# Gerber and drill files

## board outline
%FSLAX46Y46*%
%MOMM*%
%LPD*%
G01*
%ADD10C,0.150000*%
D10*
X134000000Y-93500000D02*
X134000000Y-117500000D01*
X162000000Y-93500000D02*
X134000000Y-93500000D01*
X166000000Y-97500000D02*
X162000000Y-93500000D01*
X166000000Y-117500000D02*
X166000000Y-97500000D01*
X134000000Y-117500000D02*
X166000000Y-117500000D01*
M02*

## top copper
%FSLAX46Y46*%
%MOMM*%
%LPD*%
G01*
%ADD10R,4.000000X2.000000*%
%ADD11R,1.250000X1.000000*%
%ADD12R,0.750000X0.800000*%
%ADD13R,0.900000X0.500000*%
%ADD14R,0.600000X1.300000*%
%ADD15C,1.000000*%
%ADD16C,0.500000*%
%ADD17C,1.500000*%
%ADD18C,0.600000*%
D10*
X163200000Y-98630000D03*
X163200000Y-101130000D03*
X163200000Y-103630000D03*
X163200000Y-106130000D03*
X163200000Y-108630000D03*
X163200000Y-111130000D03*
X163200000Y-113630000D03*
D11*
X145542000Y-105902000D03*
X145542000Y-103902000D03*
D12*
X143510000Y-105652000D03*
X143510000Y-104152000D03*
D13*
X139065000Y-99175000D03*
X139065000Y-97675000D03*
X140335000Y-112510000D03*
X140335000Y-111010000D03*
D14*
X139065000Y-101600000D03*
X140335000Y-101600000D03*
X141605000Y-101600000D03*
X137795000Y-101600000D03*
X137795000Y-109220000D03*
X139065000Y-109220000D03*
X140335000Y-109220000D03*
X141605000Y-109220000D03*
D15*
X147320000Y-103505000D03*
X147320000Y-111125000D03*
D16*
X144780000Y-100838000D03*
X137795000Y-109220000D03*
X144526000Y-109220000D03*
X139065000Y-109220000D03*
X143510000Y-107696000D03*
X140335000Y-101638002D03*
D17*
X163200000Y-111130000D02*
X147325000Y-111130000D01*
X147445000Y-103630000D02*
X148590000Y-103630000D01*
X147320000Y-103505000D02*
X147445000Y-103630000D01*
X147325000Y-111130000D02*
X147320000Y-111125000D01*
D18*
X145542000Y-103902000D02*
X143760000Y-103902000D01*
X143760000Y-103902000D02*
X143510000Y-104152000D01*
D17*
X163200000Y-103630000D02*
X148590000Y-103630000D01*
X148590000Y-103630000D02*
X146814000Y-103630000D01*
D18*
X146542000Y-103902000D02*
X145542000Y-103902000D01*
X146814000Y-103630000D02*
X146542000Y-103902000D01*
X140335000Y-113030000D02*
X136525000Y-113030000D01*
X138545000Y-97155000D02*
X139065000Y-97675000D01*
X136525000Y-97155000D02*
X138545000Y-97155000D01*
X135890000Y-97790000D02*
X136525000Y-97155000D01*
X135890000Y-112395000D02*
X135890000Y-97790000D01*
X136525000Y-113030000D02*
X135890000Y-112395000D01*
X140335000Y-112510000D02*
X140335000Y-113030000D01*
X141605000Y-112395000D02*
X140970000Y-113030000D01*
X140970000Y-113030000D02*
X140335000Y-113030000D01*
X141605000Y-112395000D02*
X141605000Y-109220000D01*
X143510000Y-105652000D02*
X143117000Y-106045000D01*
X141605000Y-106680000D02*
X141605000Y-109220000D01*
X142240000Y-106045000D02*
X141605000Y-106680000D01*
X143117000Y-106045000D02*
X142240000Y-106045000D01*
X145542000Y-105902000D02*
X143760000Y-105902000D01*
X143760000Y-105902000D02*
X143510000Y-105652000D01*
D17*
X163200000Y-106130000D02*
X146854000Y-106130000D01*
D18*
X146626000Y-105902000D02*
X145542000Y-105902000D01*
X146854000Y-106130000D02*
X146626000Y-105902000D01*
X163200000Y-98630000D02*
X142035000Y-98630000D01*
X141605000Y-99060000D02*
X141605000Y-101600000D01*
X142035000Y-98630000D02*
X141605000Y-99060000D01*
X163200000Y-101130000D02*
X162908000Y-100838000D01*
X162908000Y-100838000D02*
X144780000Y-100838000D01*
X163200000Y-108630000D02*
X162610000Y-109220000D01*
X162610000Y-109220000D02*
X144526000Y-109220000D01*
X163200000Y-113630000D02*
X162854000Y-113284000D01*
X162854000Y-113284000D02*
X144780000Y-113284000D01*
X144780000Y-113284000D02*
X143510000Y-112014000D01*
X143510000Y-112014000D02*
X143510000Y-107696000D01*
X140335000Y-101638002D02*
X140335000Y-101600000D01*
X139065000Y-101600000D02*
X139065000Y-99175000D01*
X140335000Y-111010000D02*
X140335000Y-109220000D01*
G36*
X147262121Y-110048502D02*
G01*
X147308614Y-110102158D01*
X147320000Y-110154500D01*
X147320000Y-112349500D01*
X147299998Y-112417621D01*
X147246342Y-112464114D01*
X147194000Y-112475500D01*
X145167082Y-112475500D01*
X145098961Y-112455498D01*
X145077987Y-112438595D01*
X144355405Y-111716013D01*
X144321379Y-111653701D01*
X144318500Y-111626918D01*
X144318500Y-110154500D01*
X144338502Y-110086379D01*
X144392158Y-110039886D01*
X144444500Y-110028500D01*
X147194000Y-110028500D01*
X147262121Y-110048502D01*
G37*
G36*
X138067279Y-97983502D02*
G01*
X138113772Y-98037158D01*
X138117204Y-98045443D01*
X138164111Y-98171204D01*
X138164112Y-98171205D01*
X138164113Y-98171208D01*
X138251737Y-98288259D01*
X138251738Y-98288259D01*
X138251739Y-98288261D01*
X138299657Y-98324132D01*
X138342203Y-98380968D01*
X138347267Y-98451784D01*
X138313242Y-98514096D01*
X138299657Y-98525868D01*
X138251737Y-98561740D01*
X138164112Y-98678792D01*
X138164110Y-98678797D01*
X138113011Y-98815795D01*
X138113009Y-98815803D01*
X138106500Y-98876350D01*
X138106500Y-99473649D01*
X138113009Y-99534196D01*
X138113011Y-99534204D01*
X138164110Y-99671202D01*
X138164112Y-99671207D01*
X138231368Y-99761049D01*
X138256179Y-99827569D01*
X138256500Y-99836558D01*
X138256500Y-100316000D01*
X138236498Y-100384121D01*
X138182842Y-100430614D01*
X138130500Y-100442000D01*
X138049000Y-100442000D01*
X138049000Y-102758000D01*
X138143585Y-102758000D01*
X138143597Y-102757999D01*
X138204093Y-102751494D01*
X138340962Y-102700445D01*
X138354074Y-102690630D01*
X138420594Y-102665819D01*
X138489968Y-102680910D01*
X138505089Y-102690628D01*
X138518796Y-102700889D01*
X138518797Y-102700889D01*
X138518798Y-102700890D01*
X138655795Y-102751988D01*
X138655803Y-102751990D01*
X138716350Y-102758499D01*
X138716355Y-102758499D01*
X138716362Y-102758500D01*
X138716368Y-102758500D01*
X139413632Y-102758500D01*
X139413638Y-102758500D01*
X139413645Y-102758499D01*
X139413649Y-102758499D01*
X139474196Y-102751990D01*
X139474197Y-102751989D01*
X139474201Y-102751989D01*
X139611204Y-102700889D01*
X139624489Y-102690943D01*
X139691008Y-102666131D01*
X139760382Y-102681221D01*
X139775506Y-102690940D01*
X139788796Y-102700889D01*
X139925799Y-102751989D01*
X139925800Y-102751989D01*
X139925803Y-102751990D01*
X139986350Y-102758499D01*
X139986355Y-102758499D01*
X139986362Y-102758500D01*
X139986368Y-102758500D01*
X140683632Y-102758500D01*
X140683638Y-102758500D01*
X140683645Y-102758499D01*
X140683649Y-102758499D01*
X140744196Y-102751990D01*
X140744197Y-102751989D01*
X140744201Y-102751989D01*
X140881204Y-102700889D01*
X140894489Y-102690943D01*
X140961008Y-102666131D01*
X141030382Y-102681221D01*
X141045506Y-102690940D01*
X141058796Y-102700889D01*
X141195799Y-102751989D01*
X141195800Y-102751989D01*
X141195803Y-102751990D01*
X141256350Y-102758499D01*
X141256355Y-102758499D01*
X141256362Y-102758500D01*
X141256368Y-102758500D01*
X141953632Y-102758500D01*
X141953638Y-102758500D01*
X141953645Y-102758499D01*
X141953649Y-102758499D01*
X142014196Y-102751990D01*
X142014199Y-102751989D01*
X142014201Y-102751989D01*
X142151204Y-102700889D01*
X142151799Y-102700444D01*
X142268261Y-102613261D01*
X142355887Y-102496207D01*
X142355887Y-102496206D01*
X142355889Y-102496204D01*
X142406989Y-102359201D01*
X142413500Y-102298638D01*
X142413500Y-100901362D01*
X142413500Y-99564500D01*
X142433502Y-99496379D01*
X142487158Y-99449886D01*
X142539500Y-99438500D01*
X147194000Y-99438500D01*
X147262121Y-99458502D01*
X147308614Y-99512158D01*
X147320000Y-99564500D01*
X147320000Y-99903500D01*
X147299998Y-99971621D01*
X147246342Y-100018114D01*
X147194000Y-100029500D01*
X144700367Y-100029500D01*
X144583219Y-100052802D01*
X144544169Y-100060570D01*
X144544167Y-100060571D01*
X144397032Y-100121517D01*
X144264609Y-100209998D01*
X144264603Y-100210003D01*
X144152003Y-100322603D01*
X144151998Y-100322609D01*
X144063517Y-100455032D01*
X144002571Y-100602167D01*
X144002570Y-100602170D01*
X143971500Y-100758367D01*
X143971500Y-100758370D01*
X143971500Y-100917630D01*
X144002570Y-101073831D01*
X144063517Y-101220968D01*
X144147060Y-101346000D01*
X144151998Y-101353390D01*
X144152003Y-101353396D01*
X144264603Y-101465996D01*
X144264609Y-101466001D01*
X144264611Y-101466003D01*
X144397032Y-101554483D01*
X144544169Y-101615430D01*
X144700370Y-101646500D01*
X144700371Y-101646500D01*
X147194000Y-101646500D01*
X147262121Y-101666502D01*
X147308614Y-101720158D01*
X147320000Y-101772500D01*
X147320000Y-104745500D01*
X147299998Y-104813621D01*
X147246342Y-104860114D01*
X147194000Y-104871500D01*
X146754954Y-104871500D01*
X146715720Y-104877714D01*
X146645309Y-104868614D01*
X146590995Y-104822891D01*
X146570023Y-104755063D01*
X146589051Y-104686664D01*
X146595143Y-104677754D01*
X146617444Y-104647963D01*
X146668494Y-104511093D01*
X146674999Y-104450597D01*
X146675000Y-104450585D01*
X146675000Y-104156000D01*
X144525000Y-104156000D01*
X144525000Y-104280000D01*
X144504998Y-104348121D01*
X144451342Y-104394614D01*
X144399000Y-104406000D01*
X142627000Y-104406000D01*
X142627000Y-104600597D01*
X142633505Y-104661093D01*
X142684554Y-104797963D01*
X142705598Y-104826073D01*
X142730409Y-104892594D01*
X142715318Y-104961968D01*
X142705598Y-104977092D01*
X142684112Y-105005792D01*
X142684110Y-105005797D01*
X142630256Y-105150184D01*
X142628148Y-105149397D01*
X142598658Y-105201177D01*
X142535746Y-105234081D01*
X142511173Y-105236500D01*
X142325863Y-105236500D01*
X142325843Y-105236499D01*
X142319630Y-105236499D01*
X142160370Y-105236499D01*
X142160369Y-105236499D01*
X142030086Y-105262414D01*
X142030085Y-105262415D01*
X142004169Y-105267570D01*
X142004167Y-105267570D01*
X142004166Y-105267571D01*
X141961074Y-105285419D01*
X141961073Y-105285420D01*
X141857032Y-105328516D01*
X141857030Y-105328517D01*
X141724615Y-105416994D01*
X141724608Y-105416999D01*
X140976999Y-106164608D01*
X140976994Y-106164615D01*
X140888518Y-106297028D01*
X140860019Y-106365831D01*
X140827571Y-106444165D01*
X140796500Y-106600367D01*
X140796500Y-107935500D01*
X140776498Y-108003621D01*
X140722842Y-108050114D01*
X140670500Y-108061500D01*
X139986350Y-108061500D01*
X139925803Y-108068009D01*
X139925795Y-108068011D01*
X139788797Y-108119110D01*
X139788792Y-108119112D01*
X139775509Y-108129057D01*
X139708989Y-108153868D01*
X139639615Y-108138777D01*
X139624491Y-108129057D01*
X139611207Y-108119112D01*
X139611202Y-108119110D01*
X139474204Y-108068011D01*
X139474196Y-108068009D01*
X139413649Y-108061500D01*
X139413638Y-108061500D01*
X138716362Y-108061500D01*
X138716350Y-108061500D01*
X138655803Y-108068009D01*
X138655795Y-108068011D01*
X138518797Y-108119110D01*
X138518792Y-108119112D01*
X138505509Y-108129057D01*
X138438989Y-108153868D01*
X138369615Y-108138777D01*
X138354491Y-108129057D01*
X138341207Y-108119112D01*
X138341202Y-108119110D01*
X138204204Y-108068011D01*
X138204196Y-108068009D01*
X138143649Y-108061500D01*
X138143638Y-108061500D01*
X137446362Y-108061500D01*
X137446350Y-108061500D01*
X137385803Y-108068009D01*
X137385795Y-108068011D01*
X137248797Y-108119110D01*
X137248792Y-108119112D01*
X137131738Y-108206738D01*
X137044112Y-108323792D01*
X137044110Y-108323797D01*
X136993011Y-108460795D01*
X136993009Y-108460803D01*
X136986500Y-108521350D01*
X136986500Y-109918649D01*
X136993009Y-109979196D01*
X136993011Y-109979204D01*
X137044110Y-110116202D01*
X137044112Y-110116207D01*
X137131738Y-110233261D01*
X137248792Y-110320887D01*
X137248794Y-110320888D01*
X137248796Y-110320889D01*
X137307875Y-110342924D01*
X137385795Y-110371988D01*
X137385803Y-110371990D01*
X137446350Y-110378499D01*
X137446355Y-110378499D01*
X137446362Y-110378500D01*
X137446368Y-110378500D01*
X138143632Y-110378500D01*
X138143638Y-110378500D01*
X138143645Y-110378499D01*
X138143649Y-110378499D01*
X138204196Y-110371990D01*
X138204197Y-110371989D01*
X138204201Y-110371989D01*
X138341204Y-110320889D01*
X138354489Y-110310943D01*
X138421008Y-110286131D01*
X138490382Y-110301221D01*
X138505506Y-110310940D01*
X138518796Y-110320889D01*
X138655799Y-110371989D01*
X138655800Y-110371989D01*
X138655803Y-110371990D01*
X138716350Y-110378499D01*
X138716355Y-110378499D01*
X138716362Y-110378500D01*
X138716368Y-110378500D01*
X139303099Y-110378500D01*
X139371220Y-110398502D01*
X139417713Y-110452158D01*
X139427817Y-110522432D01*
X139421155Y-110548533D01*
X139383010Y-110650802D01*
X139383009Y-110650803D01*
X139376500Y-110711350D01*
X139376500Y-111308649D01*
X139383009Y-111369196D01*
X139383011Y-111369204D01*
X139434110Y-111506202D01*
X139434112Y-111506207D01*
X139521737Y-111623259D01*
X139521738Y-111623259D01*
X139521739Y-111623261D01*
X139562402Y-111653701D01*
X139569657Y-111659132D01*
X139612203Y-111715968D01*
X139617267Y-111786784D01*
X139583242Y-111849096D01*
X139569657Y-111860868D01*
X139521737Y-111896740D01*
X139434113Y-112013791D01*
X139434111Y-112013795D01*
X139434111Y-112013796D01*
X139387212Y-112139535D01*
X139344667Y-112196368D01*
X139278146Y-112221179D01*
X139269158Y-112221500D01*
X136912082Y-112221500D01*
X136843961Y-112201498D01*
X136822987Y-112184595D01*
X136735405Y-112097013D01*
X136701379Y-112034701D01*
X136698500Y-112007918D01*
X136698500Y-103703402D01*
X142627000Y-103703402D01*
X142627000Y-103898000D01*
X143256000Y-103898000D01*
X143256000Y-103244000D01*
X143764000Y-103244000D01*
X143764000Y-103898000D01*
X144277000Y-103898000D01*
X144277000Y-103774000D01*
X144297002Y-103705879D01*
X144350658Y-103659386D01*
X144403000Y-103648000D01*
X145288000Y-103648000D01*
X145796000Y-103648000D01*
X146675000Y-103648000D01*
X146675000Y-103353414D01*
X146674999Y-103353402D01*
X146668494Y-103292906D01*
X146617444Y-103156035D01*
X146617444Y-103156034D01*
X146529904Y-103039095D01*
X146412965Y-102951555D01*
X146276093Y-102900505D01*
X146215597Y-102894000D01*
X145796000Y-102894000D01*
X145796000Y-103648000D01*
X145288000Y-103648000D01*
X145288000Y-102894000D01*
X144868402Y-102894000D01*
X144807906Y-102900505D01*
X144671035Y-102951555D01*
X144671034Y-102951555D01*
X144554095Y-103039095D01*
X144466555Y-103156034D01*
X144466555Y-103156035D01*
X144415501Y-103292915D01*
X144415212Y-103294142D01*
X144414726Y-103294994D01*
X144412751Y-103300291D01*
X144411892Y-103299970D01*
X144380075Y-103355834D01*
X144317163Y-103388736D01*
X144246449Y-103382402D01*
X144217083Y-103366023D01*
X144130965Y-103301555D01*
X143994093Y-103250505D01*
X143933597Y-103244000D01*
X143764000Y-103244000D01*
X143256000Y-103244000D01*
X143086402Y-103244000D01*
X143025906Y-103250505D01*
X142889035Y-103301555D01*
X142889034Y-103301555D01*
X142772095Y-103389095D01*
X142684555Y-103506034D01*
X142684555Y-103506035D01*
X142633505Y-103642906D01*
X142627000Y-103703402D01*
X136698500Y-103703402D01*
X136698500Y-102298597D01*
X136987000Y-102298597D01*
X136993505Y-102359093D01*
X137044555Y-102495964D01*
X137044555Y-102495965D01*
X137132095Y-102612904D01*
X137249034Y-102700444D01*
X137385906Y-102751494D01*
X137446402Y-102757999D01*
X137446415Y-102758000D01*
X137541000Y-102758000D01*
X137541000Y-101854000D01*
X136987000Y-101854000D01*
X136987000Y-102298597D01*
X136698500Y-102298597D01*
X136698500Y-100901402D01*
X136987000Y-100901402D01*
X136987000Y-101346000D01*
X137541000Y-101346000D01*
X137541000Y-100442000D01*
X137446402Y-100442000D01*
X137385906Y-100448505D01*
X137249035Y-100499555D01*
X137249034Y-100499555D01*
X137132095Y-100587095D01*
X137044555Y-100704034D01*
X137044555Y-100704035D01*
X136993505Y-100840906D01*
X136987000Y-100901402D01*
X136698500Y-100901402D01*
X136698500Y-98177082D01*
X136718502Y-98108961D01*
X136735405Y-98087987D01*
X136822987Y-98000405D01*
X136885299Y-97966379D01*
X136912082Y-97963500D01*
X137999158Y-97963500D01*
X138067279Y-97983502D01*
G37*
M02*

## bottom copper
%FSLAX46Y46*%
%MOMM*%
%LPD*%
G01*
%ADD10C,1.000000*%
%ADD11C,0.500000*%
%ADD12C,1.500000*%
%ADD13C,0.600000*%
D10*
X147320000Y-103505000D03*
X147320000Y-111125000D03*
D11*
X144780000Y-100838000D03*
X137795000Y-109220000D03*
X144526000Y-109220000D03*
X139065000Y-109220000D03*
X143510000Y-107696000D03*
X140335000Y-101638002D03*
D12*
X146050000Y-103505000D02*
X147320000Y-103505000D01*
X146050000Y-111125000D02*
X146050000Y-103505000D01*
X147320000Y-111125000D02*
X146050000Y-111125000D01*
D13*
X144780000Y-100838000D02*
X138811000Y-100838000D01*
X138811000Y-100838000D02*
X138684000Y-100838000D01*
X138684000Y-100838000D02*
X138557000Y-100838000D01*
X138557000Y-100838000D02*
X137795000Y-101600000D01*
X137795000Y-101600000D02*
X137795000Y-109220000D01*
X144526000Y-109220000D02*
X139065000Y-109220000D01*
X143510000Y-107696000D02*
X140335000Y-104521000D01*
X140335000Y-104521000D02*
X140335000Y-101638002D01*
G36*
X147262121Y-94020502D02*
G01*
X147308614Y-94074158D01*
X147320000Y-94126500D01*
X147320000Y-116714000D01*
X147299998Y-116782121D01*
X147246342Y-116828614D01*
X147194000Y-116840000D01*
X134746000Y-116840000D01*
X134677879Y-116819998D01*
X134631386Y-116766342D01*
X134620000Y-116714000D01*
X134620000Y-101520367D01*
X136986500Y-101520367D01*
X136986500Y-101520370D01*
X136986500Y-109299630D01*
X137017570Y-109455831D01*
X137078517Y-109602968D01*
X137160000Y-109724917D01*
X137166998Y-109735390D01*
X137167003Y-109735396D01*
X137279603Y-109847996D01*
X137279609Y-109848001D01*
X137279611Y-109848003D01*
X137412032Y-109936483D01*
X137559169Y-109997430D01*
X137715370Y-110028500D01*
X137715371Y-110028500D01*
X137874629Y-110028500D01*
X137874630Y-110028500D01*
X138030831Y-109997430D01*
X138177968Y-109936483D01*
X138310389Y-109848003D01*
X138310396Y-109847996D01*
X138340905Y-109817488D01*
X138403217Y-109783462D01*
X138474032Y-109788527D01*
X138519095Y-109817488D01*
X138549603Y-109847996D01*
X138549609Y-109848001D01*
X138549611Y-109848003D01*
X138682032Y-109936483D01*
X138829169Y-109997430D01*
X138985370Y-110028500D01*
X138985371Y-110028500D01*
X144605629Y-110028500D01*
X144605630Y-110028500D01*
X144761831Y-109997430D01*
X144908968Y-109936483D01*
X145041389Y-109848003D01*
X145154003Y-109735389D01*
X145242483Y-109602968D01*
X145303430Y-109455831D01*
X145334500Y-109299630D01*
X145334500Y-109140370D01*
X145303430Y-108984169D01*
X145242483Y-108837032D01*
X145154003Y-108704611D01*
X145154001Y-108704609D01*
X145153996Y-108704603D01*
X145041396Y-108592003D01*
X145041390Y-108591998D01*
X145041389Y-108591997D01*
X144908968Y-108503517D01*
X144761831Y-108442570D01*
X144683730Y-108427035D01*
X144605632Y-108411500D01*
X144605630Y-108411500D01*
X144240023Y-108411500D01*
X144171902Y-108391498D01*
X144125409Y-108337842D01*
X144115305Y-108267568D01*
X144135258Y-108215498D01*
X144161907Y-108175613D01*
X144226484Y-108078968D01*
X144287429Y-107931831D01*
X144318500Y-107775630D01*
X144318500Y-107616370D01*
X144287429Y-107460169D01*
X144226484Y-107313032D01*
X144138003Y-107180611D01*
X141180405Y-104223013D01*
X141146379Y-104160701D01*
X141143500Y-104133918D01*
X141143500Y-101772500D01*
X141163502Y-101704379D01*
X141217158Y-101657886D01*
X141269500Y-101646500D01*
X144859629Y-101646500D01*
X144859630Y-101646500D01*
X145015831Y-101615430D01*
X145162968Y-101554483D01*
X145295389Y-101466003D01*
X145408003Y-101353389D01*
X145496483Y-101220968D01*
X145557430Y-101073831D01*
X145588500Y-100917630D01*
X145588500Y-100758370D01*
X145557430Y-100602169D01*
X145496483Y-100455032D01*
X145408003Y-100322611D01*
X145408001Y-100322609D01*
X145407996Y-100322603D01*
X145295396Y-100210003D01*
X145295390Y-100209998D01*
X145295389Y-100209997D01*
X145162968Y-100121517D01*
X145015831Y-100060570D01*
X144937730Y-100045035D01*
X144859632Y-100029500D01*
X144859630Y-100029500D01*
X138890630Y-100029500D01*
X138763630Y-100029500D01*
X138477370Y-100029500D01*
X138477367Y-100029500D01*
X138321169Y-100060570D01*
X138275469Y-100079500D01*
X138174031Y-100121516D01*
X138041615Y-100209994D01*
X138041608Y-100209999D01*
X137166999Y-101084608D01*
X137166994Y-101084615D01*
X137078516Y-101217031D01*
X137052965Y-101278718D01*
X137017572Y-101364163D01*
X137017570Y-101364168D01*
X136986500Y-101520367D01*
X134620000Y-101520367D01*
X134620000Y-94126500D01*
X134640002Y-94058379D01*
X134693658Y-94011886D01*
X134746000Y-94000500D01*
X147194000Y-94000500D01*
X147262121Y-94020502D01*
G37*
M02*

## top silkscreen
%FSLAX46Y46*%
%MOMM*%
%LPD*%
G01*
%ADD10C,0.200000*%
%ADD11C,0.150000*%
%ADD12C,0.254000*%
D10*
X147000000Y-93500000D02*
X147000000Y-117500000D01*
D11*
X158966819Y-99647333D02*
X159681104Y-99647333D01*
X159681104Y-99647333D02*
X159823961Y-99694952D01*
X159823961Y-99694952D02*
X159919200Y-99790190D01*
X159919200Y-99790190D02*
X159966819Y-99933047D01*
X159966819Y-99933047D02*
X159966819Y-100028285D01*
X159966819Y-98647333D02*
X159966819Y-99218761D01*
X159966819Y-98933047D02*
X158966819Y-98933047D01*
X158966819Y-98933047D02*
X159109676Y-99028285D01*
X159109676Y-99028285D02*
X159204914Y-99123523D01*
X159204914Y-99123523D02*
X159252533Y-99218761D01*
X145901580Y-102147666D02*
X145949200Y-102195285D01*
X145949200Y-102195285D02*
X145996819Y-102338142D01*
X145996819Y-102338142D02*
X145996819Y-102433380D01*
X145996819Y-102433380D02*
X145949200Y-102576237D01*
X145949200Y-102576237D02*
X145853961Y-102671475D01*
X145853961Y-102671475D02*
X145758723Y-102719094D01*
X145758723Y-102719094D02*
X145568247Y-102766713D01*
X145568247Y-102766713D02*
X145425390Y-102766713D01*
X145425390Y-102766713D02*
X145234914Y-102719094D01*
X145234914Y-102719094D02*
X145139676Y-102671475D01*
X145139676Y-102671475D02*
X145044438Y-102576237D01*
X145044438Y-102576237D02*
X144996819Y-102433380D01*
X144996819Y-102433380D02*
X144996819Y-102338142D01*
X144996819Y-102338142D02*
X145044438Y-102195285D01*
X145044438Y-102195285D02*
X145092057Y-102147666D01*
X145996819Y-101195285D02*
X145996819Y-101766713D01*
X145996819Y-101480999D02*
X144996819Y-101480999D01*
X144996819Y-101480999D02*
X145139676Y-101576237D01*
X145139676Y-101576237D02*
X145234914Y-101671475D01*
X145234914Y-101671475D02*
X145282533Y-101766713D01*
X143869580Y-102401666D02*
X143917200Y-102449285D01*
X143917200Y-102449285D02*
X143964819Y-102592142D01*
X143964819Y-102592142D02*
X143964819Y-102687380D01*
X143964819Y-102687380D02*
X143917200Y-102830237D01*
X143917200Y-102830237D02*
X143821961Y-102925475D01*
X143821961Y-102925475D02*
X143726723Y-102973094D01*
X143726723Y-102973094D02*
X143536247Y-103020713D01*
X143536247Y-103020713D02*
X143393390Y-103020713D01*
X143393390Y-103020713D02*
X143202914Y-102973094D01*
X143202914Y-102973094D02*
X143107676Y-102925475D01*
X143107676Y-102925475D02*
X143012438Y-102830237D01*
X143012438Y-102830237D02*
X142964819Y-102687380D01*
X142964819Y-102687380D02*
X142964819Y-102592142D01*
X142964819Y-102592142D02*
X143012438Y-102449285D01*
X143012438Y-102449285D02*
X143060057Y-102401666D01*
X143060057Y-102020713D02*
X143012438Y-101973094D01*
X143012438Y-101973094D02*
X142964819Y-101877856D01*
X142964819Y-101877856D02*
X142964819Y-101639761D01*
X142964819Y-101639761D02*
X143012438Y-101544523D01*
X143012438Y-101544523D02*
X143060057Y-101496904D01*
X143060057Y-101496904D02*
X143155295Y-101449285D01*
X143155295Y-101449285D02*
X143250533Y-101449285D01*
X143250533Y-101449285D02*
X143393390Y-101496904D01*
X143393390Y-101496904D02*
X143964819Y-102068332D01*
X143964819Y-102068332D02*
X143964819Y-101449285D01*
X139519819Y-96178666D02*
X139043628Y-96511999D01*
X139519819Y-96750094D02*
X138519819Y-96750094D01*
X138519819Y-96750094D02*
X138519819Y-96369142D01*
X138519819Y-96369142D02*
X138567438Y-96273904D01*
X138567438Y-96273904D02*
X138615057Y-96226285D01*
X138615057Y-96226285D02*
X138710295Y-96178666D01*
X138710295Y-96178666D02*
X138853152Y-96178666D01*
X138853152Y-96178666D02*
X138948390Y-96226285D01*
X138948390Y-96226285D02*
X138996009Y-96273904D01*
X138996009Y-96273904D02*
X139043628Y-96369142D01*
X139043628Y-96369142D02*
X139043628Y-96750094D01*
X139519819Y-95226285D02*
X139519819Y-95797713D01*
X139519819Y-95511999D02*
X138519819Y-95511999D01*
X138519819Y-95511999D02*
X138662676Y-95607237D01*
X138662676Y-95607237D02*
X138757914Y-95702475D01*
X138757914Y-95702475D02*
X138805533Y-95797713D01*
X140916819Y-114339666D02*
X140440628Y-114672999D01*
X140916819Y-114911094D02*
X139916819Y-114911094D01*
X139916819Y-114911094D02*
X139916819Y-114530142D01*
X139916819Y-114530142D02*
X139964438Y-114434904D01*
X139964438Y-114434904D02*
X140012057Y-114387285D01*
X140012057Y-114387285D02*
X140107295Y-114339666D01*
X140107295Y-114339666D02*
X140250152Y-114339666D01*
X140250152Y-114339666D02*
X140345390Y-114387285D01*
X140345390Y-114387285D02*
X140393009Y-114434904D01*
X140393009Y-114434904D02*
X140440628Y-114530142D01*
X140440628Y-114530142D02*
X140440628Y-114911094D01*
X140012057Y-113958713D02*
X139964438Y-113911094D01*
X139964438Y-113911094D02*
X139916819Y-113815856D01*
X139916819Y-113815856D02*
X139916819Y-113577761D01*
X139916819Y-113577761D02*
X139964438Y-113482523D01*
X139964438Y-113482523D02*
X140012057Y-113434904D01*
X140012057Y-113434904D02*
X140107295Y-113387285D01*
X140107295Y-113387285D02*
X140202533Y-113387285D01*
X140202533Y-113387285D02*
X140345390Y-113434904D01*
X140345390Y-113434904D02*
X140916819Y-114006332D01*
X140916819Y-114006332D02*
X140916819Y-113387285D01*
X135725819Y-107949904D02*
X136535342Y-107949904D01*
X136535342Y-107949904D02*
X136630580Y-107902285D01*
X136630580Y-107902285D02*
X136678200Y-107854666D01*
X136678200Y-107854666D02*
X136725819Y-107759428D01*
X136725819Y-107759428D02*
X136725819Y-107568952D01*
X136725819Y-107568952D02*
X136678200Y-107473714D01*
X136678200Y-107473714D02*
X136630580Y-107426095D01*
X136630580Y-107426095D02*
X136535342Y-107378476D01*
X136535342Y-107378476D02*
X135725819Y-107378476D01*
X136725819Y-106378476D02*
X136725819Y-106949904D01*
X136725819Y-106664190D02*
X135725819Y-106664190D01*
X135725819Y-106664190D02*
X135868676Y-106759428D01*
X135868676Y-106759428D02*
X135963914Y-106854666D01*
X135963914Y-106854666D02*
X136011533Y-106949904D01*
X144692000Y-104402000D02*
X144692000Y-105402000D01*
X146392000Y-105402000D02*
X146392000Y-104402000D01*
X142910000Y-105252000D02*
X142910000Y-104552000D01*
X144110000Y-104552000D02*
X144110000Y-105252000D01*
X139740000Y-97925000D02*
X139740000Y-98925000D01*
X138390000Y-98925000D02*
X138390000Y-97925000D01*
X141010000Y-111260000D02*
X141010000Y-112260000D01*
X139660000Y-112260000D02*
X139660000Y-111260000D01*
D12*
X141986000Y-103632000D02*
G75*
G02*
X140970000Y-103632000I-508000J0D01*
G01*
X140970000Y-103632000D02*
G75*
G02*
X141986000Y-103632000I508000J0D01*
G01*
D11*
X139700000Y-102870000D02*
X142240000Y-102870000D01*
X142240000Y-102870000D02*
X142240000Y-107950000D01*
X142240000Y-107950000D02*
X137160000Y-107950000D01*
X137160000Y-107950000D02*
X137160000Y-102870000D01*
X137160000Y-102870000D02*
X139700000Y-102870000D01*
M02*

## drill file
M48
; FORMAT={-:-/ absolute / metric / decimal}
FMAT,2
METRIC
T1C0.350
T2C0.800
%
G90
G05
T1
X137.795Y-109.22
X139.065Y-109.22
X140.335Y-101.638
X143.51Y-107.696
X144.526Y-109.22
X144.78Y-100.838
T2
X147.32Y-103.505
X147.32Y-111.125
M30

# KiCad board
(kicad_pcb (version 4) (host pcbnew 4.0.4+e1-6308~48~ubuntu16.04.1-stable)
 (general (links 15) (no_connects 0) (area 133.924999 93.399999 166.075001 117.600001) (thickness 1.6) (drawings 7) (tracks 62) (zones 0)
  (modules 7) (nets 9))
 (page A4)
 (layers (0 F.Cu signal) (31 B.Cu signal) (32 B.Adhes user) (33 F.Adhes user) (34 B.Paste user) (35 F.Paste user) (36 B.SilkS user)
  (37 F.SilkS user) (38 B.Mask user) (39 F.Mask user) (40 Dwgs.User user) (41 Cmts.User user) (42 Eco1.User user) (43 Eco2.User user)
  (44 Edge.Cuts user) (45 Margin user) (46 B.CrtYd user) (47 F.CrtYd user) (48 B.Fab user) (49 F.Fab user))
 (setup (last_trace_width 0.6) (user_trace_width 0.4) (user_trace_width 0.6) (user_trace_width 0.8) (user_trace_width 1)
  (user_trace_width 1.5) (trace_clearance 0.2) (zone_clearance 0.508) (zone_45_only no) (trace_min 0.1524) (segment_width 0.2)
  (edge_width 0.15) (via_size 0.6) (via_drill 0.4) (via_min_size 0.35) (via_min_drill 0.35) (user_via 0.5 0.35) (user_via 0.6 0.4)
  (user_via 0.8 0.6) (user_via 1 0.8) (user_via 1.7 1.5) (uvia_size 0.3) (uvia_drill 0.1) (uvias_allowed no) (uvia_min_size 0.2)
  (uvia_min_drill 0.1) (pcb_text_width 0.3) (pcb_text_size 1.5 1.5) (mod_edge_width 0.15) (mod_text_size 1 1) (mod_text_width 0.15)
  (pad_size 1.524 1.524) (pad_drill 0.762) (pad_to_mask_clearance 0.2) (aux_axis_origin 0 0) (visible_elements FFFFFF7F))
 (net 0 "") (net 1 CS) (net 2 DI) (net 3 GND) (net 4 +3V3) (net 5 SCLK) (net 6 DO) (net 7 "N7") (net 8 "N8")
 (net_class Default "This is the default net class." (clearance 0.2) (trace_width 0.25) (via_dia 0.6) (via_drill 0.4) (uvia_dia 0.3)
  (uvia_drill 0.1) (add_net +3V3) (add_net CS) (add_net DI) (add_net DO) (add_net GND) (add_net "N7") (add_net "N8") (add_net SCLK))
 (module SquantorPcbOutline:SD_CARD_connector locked (layer F.Cu) (at 163.2 106.13)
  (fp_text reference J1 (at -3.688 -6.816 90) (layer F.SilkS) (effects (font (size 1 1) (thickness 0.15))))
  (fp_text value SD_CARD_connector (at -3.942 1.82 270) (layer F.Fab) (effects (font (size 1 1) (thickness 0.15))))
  (pad 1 smd rect (at 0 -7.5 90) (size 2 4) (layers F.Cu F.Paste F.Mask) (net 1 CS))
  (pad 2 smd rect (at 0 -5 90) (size 2 4) (layers F.Cu F.Paste F.Mask) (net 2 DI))
  (pad 3 smd rect (at 0 -2.5 90) (size 2 4) (layers F.Cu F.Paste F.Mask) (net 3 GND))
  (pad 4 smd rect (at 0 0 90) (size 2 4) (layers F.Cu F.Paste F.Mask) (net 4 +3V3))
  (pad 5 smd rect (at 0 2.5 90) (size 2 4) (layers F.Cu F.Paste F.Mask) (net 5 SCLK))
  (pad 6 smd rect (at 0 5 90) (size 2 4) (layers F.Cu F.Paste F.Mask) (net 3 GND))
  (pad 7 smd rect (at 0 7.5 90) (size 2 4) (layers F.Cu F.Paste F.Mask) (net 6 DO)))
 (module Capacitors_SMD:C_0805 (layer F.Cu) (at 145.542 104.902 90)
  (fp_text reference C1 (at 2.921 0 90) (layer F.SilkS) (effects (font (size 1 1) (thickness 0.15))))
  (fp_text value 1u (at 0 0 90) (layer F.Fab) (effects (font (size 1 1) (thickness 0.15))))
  (fp_line (start 0.5 -0.85) (end -0.5 -0.85) (layer F.SilkS) (width 0.15))
  (fp_line (start -0.5 0.85) (end 0.5 0.85) (layer F.SilkS) (width 0.15))
  (pad 1 smd rect (at -1 0 90) (size 1 1.25) (layers F.Cu F.Paste F.Mask) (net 4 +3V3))
  (pad 2 smd rect (at 1 0 90) (size 1 1.25) (layers F.Cu F.Paste F.Mask) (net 3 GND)))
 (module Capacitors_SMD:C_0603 (layer F.Cu) (at 143.51 104.902 90)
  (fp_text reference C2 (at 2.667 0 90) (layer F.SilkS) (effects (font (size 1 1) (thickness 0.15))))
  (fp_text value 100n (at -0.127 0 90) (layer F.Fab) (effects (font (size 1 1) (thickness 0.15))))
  (fp_line (start -0.35 -0.6) (end 0.35 -0.6) (layer F.SilkS) (width 0.15))
  (fp_line (start 0.35 0.6) (end -0.35 0.6) (layer F.SilkS) (width 0.15))
  (pad 1 smd rect (at -0.75 0 90) (size 0.8 0.75) (layers F.Cu F.Paste F.Mask) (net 4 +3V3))
  (pad 2 smd rect (at 0.75 0 90) (size 0.8 0.75) (layers F.Cu F.Paste F.Mask) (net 3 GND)))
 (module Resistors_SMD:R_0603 (layer F.Cu) (at 139.065 98.425 90)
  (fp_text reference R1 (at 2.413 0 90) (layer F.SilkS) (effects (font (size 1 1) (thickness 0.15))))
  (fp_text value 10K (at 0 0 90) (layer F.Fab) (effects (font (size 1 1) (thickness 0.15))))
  (fp_line (start 0.5 0.675) (end -0.5 0.675) (layer F.SilkS) (width 0.15))
  (fp_line (start -0.5 -0.675) (end 0.5 -0.675) (layer F.SilkS) (width 0.15))
  (pad 1 smd rect (at -0.75 0 90) (size 0.5 0.9) (layers F.Cu F.Paste F.Mask) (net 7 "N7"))
  (pad 2 smd rect (at 0.75 0 90) (size 0.5 0.9) (layers F.Cu F.Paste F.Mask) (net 4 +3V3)))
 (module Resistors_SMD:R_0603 (layer F.Cu) (at 140.335 111.76 90)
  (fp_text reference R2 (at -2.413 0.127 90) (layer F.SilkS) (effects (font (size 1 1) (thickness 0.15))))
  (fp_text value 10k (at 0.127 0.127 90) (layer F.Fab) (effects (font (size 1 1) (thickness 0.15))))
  (fp_line (start 0.5 0.675) (end -0.5 0.675) (layer F.SilkS) (width 0.15))
  (fp_line (start -0.5 -0.675) (end 0.5 -0.675) (layer F.SilkS) (width 0.15))
  (pad 1 smd rect (at -0.75 0 90) (size 0.5 0.9) (layers F.Cu F.Paste F.Mask) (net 4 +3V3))
  (pad 2 smd rect (at 0.75 0 90) (size 0.5 0.9) (layers F.Cu F.Paste F.Mask) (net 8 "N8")))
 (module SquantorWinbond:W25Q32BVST (layer F.Cu) (at 139.7 105.41 270)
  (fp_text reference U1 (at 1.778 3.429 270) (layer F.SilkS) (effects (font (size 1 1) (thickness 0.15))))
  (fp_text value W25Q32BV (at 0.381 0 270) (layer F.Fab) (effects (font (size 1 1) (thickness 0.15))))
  (fp_circle (center -1.778 -1.778) (end -1.27 -1.778) (layer F.SilkS) (width 0.254))
  (fp_line (start -2.54 0) (end -2.54 -2.54) (layer F.SilkS) (width 0.15))
  (fp_line (start -2.54 -2.54) (end 2.54 -2.54) (layer F.SilkS) (width 0.15))
  (fp_line (start 2.54 -2.54) (end 2.54 2.54) (layer F.SilkS) (width 0.15))
  (fp_line (start 2.54 2.54) (end -2.54 2.54) (layer F.SilkS) (width 0.15))
  (fp_line (start -2.54 2.54) (end -2.54 0) (layer F.SilkS) (width 0.15))
  (pad 3 smd rect (at -3.81 0.635 270) (size 1.3 0.6) (layers F.Cu F.Paste F.Mask) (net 7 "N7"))
  (pad 2 smd rect (at -3.81 -0.635 270) (size 1.3 0.6) (layers F.Cu F.Paste F.Mask) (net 6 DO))
  (pad 1 smd rect (at -3.81 -1.905 270) (size 1.3 0.6) (layers F.Cu F.Paste F.Mask) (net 1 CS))
  (pad 4 smd rect (at -3.81 1.905 270) (size 1.3 0.6) (layers F.Cu F.Paste F.Mask) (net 3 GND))
  (pad 5 smd rect (at 3.81 1.905 270) (size 1.3 0.6) (layers F.Cu F.Paste F.Mask) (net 2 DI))
  (pad 6 smd rect (at 3.81 0.635 270) (size 1.3 0.6) (layers F.Cu F.Paste F.Mask) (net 5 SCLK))
  (pad 7 smd rect (at 3.81 -0.635 270) (size 1.3 0.6) (layers F.Cu F.Paste F.Mask) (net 8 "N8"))
  (pad 8 smd rect (at 3.81 -1.905 270) (size 1.3 0.6) (layers F.Cu F.Paste F.Mask) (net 4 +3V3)))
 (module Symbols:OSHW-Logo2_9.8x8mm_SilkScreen (layer B.Cu) (at 142.494 104.775 270)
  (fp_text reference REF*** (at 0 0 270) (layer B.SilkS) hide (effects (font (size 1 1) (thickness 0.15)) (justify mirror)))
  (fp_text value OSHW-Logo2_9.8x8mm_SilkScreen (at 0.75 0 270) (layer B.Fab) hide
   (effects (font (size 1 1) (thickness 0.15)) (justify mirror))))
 (gr_line (start 147 93.5) (end 147 117.5) (angle 90) (layer F.SilkS) (width 0.2))
 (gr_line (start 134 93.5) (end 134 117.5) (angle 90) (layer Edge.Cuts) (width 0.15))
 (gr_line (start 162 93.5) (end 134 93.5) (angle 90) (layer Edge.Cuts) (width 0.15))
 (gr_line (start 166 97.5) (end 162 93.5) (angle 90) (layer Edge.Cuts) (width 0.15))
 (gr_line (start 166 117.5) (end 166 97.5) (angle 90) (layer Edge.Cuts) (width 0.15))
 (gr_line (start 134 117.5) (end 166 117.5) (angle 90) (layer Edge.Cuts) (width 0.15))
 (segment (start 163.2 111.13) (end 147.325 111.13) (width 1.5) (layer F.Cu) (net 3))
 (segment (start 147.445 103.63) (end 148.59 103.63) (width 1.5) (layer F.Cu) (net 3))
 (segment (start 147.32 103.505) (end 147.445 103.63) (width 1.5) (layer F.Cu) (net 3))
 (via (at 147.32 103.505) (size 1) (drill 0.8) (layers F.Cu B.Cu) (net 3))
 (segment (start 146.05 103.505) (end 147.32 103.505) (width 1.5) (layer B.Cu) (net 3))
 (segment (start 146.05 111.125) (end 146.05 103.505) (width 1.5) (layer B.Cu) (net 3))
 (segment (start 147.32 111.125) (end 146.05 111.125) (width 1.5) (layer B.Cu) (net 3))
 (via (at 147.32 111.125) (size 1) (drill 0.8) (layers F.Cu B.Cu) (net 3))
 (segment (start 147.325 111.13) (end 147.32 111.125) (width 1.5) (layer F.Cu) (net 3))
 (segment (start 145.542 103.902) (end 143.76 103.902) (width 0.6) (layer F.Cu) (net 3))
 (segment (start 143.76 103.902) (end 143.51 104.152) (width 0.6) (layer F.Cu) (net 3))
 (segment (start 163.2 103.63) (end 148.59 103.63) (width 1.5) (layer F.Cu) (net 3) (status 10))
 (segment (start 148.59 103.63) (end 146.814 103.63) (width 1.5) (layer F.Cu) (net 3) (status 10))
 (segment (start 146.542 103.902) (end 145.542 103.902) (width 0.6) (layer F.Cu) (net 3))
 (segment (start 146.814 103.63) (end 146.542 103.902) (width 0.6) (layer F.Cu) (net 3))
 (segment (start 140.335 113.03) (end 136.525 113.03) (width 0.6) (layer F.Cu) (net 4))
 (segment (start 138.545 97.155) (end 139.065 97.675) (width 0.6) (layer F.Cu) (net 4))
 (segment (start 136.525 97.155) (end 138.545 97.155) (width 0.6) (layer F.Cu) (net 4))
 (segment (start 135.89 97.79) (end 136.525 97.155) (width 0.6) (layer F.Cu) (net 4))
 (segment (start 135.89 112.395) (end 135.89 97.79) (width 0.6) (layer F.Cu) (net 4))
 (segment (start 136.525 113.03) (end 135.89 112.395) (width 0.6) (layer F.Cu) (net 4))
 (segment (start 140.335 112.51) (end 140.335 113.03) (width 0.6) (layer F.Cu) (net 4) (status 10))
 (segment (start 141.605 112.395) (end 140.97 113.03) (width 0.6) (layer F.Cu) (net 4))
 (segment (start 140.97 113.03) (end 140.335 113.03) (width 0.6) (layer F.Cu) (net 4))
 (segment (start 141.605 112.395) (end 141.605 109.22) (width 0.6) (layer F.Cu) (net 4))
 (segment (start 143.51 105.652) (end 143.117 106.045) (width 0.6) (layer F.Cu) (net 4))
 (segment (start 141.605 106.68) (end 141.605 109.22) (width 0.6) (layer F.Cu) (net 4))
 (segment (start 142.24 106.045) (end 141.605 106.68) (width 0.6) (layer F.Cu) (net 4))
 (segment (start 143.117 106.045) (end 142.24 106.045) (width 0.6) (layer F.Cu) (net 4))
 (segment (start 145.542 105.902) (end 143.76 105.902) (width 0.6) (layer F.Cu) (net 4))
 (segment (start 143.76 105.902) (end 143.51 105.652) (width 0.6) (layer F.Cu) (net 4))
 (segment (start 163.2 106.13) (end 146.854 106.13) (width 1.5) (layer F.Cu) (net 4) (status 10))
 (segment (start 146.626 105.902) (end 145.542 105.902) (width 0.6) (layer F.Cu) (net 4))
 (segment (start 146.854 106.13) (end 146.626 105.902) (width 0.6) (layer F.Cu) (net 4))
 (segment (start 163.2 98.63) (end 142.035 98.63) (width 0.6) (layer F.Cu) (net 1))
 (segment (start 141.605 99.06) (end 141.605 101.6) (width 0.6) (layer F.Cu) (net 1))
 (segment (start 142.035 98.63) (end 141.605 99.06) (width 0.6) (layer F.Cu) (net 1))
 (segment (start 163.2 101.13) (end 162.908 100.838) (width 0.6) (layer F.Cu) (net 2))
 (segment (start 162.908 100.838) (end 144.78 100.838) (width 0.6) (layer F.Cu) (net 2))
 (via (at 144.78 100.838) (size 0.5) (drill 0.35) (layers F.Cu B.Cu) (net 2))
 (segment (start 144.78 100.838) (end 138.811 100.838) (width 0.6) (layer B.Cu) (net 2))
 (segment (start 138.811 100.838) (end 138.684 100.838) (width 0.6) (layer B.Cu) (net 2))
 (segment (start 138.684 100.838) (end 138.557 100.838) (width 0.6) (layer B.Cu) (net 2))
 (segment (start 138.557 100.838) (end 137.795 101.6) (width 0.6) (layer B.Cu) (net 2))
 (segment (start 137.795 101.6) (end 137.795 109.22) (width 0.6) (layer B.Cu) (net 2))
 (via (at 137.795 109.22) (size 0.5) (drill 0.35) (layers F.Cu B.Cu) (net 2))
 (segment (start 163.2 108.63) (end 162.61 109.22) (width 0.6) (layer F.Cu) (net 5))
 (segment (start 162.61 109.22) (end 144.526 109.22) (width 0.6) (layer F.Cu) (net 5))
 (via (at 144.526 109.22) (size 0.5) (drill 0.35) (layers F.Cu B.Cu) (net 5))
 (segment (start 144.526 109.22) (end 139.065 109.22) (width 0.6) (layer B.Cu) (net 5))
 (via (at 139.065 109.22) (size 0.5) (drill 0.35) (layers F.Cu B.Cu) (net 5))
 (segment (start 163.2 113.63) (end 162.854 113.284) (width 0.6) (layer F.Cu) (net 6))
 (segment (start 162.854 113.284) (end 144.78 113.284) (width 0.6) (layer F.Cu) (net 6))
 (segment (start 144.78 113.284) (end 143.51 112.014) (width 0.6) (layer F.Cu) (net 6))
 (segment (start 143.51 112.014) (end 143.51 107.696) (width 0.6) (layer F.Cu) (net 6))
 (via (at 143.51 107.696) (size 0.5) (drill 0.35) (layers F.Cu B.Cu) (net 6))
 (segment (start 143.51 107.696) (end 140.335 104.521) (width 0.6) (layer B.Cu) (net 6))
 (segment (start 140.335 104.521) (end 140.335 101.638002) (width 0.6) (layer B.Cu) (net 6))
 (via (at 140.335 101.638002) (size 0.5) (drill 0.35) (layers F.Cu B.Cu) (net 6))
 (segment (start 140.335 101.638002) (end 140.335 101.6) (width 0.6) (layer F.Cu) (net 6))
 (segment (start 139.065 101.6) (end 139.065 99.175) (width 0.6) (layer F.Cu) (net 7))
 (segment (start 140.335 111.01) (end 140.335 109.22) (width 0.6) (layer F.Cu) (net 8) (status 10))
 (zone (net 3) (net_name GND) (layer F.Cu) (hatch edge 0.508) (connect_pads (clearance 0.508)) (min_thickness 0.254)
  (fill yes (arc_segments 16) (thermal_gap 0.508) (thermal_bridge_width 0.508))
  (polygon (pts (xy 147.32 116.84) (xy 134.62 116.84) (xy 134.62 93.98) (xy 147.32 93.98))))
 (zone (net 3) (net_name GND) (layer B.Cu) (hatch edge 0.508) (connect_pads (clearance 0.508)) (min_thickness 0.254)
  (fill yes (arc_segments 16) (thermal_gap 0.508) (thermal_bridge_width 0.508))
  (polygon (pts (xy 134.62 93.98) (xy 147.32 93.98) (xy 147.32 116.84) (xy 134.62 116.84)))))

